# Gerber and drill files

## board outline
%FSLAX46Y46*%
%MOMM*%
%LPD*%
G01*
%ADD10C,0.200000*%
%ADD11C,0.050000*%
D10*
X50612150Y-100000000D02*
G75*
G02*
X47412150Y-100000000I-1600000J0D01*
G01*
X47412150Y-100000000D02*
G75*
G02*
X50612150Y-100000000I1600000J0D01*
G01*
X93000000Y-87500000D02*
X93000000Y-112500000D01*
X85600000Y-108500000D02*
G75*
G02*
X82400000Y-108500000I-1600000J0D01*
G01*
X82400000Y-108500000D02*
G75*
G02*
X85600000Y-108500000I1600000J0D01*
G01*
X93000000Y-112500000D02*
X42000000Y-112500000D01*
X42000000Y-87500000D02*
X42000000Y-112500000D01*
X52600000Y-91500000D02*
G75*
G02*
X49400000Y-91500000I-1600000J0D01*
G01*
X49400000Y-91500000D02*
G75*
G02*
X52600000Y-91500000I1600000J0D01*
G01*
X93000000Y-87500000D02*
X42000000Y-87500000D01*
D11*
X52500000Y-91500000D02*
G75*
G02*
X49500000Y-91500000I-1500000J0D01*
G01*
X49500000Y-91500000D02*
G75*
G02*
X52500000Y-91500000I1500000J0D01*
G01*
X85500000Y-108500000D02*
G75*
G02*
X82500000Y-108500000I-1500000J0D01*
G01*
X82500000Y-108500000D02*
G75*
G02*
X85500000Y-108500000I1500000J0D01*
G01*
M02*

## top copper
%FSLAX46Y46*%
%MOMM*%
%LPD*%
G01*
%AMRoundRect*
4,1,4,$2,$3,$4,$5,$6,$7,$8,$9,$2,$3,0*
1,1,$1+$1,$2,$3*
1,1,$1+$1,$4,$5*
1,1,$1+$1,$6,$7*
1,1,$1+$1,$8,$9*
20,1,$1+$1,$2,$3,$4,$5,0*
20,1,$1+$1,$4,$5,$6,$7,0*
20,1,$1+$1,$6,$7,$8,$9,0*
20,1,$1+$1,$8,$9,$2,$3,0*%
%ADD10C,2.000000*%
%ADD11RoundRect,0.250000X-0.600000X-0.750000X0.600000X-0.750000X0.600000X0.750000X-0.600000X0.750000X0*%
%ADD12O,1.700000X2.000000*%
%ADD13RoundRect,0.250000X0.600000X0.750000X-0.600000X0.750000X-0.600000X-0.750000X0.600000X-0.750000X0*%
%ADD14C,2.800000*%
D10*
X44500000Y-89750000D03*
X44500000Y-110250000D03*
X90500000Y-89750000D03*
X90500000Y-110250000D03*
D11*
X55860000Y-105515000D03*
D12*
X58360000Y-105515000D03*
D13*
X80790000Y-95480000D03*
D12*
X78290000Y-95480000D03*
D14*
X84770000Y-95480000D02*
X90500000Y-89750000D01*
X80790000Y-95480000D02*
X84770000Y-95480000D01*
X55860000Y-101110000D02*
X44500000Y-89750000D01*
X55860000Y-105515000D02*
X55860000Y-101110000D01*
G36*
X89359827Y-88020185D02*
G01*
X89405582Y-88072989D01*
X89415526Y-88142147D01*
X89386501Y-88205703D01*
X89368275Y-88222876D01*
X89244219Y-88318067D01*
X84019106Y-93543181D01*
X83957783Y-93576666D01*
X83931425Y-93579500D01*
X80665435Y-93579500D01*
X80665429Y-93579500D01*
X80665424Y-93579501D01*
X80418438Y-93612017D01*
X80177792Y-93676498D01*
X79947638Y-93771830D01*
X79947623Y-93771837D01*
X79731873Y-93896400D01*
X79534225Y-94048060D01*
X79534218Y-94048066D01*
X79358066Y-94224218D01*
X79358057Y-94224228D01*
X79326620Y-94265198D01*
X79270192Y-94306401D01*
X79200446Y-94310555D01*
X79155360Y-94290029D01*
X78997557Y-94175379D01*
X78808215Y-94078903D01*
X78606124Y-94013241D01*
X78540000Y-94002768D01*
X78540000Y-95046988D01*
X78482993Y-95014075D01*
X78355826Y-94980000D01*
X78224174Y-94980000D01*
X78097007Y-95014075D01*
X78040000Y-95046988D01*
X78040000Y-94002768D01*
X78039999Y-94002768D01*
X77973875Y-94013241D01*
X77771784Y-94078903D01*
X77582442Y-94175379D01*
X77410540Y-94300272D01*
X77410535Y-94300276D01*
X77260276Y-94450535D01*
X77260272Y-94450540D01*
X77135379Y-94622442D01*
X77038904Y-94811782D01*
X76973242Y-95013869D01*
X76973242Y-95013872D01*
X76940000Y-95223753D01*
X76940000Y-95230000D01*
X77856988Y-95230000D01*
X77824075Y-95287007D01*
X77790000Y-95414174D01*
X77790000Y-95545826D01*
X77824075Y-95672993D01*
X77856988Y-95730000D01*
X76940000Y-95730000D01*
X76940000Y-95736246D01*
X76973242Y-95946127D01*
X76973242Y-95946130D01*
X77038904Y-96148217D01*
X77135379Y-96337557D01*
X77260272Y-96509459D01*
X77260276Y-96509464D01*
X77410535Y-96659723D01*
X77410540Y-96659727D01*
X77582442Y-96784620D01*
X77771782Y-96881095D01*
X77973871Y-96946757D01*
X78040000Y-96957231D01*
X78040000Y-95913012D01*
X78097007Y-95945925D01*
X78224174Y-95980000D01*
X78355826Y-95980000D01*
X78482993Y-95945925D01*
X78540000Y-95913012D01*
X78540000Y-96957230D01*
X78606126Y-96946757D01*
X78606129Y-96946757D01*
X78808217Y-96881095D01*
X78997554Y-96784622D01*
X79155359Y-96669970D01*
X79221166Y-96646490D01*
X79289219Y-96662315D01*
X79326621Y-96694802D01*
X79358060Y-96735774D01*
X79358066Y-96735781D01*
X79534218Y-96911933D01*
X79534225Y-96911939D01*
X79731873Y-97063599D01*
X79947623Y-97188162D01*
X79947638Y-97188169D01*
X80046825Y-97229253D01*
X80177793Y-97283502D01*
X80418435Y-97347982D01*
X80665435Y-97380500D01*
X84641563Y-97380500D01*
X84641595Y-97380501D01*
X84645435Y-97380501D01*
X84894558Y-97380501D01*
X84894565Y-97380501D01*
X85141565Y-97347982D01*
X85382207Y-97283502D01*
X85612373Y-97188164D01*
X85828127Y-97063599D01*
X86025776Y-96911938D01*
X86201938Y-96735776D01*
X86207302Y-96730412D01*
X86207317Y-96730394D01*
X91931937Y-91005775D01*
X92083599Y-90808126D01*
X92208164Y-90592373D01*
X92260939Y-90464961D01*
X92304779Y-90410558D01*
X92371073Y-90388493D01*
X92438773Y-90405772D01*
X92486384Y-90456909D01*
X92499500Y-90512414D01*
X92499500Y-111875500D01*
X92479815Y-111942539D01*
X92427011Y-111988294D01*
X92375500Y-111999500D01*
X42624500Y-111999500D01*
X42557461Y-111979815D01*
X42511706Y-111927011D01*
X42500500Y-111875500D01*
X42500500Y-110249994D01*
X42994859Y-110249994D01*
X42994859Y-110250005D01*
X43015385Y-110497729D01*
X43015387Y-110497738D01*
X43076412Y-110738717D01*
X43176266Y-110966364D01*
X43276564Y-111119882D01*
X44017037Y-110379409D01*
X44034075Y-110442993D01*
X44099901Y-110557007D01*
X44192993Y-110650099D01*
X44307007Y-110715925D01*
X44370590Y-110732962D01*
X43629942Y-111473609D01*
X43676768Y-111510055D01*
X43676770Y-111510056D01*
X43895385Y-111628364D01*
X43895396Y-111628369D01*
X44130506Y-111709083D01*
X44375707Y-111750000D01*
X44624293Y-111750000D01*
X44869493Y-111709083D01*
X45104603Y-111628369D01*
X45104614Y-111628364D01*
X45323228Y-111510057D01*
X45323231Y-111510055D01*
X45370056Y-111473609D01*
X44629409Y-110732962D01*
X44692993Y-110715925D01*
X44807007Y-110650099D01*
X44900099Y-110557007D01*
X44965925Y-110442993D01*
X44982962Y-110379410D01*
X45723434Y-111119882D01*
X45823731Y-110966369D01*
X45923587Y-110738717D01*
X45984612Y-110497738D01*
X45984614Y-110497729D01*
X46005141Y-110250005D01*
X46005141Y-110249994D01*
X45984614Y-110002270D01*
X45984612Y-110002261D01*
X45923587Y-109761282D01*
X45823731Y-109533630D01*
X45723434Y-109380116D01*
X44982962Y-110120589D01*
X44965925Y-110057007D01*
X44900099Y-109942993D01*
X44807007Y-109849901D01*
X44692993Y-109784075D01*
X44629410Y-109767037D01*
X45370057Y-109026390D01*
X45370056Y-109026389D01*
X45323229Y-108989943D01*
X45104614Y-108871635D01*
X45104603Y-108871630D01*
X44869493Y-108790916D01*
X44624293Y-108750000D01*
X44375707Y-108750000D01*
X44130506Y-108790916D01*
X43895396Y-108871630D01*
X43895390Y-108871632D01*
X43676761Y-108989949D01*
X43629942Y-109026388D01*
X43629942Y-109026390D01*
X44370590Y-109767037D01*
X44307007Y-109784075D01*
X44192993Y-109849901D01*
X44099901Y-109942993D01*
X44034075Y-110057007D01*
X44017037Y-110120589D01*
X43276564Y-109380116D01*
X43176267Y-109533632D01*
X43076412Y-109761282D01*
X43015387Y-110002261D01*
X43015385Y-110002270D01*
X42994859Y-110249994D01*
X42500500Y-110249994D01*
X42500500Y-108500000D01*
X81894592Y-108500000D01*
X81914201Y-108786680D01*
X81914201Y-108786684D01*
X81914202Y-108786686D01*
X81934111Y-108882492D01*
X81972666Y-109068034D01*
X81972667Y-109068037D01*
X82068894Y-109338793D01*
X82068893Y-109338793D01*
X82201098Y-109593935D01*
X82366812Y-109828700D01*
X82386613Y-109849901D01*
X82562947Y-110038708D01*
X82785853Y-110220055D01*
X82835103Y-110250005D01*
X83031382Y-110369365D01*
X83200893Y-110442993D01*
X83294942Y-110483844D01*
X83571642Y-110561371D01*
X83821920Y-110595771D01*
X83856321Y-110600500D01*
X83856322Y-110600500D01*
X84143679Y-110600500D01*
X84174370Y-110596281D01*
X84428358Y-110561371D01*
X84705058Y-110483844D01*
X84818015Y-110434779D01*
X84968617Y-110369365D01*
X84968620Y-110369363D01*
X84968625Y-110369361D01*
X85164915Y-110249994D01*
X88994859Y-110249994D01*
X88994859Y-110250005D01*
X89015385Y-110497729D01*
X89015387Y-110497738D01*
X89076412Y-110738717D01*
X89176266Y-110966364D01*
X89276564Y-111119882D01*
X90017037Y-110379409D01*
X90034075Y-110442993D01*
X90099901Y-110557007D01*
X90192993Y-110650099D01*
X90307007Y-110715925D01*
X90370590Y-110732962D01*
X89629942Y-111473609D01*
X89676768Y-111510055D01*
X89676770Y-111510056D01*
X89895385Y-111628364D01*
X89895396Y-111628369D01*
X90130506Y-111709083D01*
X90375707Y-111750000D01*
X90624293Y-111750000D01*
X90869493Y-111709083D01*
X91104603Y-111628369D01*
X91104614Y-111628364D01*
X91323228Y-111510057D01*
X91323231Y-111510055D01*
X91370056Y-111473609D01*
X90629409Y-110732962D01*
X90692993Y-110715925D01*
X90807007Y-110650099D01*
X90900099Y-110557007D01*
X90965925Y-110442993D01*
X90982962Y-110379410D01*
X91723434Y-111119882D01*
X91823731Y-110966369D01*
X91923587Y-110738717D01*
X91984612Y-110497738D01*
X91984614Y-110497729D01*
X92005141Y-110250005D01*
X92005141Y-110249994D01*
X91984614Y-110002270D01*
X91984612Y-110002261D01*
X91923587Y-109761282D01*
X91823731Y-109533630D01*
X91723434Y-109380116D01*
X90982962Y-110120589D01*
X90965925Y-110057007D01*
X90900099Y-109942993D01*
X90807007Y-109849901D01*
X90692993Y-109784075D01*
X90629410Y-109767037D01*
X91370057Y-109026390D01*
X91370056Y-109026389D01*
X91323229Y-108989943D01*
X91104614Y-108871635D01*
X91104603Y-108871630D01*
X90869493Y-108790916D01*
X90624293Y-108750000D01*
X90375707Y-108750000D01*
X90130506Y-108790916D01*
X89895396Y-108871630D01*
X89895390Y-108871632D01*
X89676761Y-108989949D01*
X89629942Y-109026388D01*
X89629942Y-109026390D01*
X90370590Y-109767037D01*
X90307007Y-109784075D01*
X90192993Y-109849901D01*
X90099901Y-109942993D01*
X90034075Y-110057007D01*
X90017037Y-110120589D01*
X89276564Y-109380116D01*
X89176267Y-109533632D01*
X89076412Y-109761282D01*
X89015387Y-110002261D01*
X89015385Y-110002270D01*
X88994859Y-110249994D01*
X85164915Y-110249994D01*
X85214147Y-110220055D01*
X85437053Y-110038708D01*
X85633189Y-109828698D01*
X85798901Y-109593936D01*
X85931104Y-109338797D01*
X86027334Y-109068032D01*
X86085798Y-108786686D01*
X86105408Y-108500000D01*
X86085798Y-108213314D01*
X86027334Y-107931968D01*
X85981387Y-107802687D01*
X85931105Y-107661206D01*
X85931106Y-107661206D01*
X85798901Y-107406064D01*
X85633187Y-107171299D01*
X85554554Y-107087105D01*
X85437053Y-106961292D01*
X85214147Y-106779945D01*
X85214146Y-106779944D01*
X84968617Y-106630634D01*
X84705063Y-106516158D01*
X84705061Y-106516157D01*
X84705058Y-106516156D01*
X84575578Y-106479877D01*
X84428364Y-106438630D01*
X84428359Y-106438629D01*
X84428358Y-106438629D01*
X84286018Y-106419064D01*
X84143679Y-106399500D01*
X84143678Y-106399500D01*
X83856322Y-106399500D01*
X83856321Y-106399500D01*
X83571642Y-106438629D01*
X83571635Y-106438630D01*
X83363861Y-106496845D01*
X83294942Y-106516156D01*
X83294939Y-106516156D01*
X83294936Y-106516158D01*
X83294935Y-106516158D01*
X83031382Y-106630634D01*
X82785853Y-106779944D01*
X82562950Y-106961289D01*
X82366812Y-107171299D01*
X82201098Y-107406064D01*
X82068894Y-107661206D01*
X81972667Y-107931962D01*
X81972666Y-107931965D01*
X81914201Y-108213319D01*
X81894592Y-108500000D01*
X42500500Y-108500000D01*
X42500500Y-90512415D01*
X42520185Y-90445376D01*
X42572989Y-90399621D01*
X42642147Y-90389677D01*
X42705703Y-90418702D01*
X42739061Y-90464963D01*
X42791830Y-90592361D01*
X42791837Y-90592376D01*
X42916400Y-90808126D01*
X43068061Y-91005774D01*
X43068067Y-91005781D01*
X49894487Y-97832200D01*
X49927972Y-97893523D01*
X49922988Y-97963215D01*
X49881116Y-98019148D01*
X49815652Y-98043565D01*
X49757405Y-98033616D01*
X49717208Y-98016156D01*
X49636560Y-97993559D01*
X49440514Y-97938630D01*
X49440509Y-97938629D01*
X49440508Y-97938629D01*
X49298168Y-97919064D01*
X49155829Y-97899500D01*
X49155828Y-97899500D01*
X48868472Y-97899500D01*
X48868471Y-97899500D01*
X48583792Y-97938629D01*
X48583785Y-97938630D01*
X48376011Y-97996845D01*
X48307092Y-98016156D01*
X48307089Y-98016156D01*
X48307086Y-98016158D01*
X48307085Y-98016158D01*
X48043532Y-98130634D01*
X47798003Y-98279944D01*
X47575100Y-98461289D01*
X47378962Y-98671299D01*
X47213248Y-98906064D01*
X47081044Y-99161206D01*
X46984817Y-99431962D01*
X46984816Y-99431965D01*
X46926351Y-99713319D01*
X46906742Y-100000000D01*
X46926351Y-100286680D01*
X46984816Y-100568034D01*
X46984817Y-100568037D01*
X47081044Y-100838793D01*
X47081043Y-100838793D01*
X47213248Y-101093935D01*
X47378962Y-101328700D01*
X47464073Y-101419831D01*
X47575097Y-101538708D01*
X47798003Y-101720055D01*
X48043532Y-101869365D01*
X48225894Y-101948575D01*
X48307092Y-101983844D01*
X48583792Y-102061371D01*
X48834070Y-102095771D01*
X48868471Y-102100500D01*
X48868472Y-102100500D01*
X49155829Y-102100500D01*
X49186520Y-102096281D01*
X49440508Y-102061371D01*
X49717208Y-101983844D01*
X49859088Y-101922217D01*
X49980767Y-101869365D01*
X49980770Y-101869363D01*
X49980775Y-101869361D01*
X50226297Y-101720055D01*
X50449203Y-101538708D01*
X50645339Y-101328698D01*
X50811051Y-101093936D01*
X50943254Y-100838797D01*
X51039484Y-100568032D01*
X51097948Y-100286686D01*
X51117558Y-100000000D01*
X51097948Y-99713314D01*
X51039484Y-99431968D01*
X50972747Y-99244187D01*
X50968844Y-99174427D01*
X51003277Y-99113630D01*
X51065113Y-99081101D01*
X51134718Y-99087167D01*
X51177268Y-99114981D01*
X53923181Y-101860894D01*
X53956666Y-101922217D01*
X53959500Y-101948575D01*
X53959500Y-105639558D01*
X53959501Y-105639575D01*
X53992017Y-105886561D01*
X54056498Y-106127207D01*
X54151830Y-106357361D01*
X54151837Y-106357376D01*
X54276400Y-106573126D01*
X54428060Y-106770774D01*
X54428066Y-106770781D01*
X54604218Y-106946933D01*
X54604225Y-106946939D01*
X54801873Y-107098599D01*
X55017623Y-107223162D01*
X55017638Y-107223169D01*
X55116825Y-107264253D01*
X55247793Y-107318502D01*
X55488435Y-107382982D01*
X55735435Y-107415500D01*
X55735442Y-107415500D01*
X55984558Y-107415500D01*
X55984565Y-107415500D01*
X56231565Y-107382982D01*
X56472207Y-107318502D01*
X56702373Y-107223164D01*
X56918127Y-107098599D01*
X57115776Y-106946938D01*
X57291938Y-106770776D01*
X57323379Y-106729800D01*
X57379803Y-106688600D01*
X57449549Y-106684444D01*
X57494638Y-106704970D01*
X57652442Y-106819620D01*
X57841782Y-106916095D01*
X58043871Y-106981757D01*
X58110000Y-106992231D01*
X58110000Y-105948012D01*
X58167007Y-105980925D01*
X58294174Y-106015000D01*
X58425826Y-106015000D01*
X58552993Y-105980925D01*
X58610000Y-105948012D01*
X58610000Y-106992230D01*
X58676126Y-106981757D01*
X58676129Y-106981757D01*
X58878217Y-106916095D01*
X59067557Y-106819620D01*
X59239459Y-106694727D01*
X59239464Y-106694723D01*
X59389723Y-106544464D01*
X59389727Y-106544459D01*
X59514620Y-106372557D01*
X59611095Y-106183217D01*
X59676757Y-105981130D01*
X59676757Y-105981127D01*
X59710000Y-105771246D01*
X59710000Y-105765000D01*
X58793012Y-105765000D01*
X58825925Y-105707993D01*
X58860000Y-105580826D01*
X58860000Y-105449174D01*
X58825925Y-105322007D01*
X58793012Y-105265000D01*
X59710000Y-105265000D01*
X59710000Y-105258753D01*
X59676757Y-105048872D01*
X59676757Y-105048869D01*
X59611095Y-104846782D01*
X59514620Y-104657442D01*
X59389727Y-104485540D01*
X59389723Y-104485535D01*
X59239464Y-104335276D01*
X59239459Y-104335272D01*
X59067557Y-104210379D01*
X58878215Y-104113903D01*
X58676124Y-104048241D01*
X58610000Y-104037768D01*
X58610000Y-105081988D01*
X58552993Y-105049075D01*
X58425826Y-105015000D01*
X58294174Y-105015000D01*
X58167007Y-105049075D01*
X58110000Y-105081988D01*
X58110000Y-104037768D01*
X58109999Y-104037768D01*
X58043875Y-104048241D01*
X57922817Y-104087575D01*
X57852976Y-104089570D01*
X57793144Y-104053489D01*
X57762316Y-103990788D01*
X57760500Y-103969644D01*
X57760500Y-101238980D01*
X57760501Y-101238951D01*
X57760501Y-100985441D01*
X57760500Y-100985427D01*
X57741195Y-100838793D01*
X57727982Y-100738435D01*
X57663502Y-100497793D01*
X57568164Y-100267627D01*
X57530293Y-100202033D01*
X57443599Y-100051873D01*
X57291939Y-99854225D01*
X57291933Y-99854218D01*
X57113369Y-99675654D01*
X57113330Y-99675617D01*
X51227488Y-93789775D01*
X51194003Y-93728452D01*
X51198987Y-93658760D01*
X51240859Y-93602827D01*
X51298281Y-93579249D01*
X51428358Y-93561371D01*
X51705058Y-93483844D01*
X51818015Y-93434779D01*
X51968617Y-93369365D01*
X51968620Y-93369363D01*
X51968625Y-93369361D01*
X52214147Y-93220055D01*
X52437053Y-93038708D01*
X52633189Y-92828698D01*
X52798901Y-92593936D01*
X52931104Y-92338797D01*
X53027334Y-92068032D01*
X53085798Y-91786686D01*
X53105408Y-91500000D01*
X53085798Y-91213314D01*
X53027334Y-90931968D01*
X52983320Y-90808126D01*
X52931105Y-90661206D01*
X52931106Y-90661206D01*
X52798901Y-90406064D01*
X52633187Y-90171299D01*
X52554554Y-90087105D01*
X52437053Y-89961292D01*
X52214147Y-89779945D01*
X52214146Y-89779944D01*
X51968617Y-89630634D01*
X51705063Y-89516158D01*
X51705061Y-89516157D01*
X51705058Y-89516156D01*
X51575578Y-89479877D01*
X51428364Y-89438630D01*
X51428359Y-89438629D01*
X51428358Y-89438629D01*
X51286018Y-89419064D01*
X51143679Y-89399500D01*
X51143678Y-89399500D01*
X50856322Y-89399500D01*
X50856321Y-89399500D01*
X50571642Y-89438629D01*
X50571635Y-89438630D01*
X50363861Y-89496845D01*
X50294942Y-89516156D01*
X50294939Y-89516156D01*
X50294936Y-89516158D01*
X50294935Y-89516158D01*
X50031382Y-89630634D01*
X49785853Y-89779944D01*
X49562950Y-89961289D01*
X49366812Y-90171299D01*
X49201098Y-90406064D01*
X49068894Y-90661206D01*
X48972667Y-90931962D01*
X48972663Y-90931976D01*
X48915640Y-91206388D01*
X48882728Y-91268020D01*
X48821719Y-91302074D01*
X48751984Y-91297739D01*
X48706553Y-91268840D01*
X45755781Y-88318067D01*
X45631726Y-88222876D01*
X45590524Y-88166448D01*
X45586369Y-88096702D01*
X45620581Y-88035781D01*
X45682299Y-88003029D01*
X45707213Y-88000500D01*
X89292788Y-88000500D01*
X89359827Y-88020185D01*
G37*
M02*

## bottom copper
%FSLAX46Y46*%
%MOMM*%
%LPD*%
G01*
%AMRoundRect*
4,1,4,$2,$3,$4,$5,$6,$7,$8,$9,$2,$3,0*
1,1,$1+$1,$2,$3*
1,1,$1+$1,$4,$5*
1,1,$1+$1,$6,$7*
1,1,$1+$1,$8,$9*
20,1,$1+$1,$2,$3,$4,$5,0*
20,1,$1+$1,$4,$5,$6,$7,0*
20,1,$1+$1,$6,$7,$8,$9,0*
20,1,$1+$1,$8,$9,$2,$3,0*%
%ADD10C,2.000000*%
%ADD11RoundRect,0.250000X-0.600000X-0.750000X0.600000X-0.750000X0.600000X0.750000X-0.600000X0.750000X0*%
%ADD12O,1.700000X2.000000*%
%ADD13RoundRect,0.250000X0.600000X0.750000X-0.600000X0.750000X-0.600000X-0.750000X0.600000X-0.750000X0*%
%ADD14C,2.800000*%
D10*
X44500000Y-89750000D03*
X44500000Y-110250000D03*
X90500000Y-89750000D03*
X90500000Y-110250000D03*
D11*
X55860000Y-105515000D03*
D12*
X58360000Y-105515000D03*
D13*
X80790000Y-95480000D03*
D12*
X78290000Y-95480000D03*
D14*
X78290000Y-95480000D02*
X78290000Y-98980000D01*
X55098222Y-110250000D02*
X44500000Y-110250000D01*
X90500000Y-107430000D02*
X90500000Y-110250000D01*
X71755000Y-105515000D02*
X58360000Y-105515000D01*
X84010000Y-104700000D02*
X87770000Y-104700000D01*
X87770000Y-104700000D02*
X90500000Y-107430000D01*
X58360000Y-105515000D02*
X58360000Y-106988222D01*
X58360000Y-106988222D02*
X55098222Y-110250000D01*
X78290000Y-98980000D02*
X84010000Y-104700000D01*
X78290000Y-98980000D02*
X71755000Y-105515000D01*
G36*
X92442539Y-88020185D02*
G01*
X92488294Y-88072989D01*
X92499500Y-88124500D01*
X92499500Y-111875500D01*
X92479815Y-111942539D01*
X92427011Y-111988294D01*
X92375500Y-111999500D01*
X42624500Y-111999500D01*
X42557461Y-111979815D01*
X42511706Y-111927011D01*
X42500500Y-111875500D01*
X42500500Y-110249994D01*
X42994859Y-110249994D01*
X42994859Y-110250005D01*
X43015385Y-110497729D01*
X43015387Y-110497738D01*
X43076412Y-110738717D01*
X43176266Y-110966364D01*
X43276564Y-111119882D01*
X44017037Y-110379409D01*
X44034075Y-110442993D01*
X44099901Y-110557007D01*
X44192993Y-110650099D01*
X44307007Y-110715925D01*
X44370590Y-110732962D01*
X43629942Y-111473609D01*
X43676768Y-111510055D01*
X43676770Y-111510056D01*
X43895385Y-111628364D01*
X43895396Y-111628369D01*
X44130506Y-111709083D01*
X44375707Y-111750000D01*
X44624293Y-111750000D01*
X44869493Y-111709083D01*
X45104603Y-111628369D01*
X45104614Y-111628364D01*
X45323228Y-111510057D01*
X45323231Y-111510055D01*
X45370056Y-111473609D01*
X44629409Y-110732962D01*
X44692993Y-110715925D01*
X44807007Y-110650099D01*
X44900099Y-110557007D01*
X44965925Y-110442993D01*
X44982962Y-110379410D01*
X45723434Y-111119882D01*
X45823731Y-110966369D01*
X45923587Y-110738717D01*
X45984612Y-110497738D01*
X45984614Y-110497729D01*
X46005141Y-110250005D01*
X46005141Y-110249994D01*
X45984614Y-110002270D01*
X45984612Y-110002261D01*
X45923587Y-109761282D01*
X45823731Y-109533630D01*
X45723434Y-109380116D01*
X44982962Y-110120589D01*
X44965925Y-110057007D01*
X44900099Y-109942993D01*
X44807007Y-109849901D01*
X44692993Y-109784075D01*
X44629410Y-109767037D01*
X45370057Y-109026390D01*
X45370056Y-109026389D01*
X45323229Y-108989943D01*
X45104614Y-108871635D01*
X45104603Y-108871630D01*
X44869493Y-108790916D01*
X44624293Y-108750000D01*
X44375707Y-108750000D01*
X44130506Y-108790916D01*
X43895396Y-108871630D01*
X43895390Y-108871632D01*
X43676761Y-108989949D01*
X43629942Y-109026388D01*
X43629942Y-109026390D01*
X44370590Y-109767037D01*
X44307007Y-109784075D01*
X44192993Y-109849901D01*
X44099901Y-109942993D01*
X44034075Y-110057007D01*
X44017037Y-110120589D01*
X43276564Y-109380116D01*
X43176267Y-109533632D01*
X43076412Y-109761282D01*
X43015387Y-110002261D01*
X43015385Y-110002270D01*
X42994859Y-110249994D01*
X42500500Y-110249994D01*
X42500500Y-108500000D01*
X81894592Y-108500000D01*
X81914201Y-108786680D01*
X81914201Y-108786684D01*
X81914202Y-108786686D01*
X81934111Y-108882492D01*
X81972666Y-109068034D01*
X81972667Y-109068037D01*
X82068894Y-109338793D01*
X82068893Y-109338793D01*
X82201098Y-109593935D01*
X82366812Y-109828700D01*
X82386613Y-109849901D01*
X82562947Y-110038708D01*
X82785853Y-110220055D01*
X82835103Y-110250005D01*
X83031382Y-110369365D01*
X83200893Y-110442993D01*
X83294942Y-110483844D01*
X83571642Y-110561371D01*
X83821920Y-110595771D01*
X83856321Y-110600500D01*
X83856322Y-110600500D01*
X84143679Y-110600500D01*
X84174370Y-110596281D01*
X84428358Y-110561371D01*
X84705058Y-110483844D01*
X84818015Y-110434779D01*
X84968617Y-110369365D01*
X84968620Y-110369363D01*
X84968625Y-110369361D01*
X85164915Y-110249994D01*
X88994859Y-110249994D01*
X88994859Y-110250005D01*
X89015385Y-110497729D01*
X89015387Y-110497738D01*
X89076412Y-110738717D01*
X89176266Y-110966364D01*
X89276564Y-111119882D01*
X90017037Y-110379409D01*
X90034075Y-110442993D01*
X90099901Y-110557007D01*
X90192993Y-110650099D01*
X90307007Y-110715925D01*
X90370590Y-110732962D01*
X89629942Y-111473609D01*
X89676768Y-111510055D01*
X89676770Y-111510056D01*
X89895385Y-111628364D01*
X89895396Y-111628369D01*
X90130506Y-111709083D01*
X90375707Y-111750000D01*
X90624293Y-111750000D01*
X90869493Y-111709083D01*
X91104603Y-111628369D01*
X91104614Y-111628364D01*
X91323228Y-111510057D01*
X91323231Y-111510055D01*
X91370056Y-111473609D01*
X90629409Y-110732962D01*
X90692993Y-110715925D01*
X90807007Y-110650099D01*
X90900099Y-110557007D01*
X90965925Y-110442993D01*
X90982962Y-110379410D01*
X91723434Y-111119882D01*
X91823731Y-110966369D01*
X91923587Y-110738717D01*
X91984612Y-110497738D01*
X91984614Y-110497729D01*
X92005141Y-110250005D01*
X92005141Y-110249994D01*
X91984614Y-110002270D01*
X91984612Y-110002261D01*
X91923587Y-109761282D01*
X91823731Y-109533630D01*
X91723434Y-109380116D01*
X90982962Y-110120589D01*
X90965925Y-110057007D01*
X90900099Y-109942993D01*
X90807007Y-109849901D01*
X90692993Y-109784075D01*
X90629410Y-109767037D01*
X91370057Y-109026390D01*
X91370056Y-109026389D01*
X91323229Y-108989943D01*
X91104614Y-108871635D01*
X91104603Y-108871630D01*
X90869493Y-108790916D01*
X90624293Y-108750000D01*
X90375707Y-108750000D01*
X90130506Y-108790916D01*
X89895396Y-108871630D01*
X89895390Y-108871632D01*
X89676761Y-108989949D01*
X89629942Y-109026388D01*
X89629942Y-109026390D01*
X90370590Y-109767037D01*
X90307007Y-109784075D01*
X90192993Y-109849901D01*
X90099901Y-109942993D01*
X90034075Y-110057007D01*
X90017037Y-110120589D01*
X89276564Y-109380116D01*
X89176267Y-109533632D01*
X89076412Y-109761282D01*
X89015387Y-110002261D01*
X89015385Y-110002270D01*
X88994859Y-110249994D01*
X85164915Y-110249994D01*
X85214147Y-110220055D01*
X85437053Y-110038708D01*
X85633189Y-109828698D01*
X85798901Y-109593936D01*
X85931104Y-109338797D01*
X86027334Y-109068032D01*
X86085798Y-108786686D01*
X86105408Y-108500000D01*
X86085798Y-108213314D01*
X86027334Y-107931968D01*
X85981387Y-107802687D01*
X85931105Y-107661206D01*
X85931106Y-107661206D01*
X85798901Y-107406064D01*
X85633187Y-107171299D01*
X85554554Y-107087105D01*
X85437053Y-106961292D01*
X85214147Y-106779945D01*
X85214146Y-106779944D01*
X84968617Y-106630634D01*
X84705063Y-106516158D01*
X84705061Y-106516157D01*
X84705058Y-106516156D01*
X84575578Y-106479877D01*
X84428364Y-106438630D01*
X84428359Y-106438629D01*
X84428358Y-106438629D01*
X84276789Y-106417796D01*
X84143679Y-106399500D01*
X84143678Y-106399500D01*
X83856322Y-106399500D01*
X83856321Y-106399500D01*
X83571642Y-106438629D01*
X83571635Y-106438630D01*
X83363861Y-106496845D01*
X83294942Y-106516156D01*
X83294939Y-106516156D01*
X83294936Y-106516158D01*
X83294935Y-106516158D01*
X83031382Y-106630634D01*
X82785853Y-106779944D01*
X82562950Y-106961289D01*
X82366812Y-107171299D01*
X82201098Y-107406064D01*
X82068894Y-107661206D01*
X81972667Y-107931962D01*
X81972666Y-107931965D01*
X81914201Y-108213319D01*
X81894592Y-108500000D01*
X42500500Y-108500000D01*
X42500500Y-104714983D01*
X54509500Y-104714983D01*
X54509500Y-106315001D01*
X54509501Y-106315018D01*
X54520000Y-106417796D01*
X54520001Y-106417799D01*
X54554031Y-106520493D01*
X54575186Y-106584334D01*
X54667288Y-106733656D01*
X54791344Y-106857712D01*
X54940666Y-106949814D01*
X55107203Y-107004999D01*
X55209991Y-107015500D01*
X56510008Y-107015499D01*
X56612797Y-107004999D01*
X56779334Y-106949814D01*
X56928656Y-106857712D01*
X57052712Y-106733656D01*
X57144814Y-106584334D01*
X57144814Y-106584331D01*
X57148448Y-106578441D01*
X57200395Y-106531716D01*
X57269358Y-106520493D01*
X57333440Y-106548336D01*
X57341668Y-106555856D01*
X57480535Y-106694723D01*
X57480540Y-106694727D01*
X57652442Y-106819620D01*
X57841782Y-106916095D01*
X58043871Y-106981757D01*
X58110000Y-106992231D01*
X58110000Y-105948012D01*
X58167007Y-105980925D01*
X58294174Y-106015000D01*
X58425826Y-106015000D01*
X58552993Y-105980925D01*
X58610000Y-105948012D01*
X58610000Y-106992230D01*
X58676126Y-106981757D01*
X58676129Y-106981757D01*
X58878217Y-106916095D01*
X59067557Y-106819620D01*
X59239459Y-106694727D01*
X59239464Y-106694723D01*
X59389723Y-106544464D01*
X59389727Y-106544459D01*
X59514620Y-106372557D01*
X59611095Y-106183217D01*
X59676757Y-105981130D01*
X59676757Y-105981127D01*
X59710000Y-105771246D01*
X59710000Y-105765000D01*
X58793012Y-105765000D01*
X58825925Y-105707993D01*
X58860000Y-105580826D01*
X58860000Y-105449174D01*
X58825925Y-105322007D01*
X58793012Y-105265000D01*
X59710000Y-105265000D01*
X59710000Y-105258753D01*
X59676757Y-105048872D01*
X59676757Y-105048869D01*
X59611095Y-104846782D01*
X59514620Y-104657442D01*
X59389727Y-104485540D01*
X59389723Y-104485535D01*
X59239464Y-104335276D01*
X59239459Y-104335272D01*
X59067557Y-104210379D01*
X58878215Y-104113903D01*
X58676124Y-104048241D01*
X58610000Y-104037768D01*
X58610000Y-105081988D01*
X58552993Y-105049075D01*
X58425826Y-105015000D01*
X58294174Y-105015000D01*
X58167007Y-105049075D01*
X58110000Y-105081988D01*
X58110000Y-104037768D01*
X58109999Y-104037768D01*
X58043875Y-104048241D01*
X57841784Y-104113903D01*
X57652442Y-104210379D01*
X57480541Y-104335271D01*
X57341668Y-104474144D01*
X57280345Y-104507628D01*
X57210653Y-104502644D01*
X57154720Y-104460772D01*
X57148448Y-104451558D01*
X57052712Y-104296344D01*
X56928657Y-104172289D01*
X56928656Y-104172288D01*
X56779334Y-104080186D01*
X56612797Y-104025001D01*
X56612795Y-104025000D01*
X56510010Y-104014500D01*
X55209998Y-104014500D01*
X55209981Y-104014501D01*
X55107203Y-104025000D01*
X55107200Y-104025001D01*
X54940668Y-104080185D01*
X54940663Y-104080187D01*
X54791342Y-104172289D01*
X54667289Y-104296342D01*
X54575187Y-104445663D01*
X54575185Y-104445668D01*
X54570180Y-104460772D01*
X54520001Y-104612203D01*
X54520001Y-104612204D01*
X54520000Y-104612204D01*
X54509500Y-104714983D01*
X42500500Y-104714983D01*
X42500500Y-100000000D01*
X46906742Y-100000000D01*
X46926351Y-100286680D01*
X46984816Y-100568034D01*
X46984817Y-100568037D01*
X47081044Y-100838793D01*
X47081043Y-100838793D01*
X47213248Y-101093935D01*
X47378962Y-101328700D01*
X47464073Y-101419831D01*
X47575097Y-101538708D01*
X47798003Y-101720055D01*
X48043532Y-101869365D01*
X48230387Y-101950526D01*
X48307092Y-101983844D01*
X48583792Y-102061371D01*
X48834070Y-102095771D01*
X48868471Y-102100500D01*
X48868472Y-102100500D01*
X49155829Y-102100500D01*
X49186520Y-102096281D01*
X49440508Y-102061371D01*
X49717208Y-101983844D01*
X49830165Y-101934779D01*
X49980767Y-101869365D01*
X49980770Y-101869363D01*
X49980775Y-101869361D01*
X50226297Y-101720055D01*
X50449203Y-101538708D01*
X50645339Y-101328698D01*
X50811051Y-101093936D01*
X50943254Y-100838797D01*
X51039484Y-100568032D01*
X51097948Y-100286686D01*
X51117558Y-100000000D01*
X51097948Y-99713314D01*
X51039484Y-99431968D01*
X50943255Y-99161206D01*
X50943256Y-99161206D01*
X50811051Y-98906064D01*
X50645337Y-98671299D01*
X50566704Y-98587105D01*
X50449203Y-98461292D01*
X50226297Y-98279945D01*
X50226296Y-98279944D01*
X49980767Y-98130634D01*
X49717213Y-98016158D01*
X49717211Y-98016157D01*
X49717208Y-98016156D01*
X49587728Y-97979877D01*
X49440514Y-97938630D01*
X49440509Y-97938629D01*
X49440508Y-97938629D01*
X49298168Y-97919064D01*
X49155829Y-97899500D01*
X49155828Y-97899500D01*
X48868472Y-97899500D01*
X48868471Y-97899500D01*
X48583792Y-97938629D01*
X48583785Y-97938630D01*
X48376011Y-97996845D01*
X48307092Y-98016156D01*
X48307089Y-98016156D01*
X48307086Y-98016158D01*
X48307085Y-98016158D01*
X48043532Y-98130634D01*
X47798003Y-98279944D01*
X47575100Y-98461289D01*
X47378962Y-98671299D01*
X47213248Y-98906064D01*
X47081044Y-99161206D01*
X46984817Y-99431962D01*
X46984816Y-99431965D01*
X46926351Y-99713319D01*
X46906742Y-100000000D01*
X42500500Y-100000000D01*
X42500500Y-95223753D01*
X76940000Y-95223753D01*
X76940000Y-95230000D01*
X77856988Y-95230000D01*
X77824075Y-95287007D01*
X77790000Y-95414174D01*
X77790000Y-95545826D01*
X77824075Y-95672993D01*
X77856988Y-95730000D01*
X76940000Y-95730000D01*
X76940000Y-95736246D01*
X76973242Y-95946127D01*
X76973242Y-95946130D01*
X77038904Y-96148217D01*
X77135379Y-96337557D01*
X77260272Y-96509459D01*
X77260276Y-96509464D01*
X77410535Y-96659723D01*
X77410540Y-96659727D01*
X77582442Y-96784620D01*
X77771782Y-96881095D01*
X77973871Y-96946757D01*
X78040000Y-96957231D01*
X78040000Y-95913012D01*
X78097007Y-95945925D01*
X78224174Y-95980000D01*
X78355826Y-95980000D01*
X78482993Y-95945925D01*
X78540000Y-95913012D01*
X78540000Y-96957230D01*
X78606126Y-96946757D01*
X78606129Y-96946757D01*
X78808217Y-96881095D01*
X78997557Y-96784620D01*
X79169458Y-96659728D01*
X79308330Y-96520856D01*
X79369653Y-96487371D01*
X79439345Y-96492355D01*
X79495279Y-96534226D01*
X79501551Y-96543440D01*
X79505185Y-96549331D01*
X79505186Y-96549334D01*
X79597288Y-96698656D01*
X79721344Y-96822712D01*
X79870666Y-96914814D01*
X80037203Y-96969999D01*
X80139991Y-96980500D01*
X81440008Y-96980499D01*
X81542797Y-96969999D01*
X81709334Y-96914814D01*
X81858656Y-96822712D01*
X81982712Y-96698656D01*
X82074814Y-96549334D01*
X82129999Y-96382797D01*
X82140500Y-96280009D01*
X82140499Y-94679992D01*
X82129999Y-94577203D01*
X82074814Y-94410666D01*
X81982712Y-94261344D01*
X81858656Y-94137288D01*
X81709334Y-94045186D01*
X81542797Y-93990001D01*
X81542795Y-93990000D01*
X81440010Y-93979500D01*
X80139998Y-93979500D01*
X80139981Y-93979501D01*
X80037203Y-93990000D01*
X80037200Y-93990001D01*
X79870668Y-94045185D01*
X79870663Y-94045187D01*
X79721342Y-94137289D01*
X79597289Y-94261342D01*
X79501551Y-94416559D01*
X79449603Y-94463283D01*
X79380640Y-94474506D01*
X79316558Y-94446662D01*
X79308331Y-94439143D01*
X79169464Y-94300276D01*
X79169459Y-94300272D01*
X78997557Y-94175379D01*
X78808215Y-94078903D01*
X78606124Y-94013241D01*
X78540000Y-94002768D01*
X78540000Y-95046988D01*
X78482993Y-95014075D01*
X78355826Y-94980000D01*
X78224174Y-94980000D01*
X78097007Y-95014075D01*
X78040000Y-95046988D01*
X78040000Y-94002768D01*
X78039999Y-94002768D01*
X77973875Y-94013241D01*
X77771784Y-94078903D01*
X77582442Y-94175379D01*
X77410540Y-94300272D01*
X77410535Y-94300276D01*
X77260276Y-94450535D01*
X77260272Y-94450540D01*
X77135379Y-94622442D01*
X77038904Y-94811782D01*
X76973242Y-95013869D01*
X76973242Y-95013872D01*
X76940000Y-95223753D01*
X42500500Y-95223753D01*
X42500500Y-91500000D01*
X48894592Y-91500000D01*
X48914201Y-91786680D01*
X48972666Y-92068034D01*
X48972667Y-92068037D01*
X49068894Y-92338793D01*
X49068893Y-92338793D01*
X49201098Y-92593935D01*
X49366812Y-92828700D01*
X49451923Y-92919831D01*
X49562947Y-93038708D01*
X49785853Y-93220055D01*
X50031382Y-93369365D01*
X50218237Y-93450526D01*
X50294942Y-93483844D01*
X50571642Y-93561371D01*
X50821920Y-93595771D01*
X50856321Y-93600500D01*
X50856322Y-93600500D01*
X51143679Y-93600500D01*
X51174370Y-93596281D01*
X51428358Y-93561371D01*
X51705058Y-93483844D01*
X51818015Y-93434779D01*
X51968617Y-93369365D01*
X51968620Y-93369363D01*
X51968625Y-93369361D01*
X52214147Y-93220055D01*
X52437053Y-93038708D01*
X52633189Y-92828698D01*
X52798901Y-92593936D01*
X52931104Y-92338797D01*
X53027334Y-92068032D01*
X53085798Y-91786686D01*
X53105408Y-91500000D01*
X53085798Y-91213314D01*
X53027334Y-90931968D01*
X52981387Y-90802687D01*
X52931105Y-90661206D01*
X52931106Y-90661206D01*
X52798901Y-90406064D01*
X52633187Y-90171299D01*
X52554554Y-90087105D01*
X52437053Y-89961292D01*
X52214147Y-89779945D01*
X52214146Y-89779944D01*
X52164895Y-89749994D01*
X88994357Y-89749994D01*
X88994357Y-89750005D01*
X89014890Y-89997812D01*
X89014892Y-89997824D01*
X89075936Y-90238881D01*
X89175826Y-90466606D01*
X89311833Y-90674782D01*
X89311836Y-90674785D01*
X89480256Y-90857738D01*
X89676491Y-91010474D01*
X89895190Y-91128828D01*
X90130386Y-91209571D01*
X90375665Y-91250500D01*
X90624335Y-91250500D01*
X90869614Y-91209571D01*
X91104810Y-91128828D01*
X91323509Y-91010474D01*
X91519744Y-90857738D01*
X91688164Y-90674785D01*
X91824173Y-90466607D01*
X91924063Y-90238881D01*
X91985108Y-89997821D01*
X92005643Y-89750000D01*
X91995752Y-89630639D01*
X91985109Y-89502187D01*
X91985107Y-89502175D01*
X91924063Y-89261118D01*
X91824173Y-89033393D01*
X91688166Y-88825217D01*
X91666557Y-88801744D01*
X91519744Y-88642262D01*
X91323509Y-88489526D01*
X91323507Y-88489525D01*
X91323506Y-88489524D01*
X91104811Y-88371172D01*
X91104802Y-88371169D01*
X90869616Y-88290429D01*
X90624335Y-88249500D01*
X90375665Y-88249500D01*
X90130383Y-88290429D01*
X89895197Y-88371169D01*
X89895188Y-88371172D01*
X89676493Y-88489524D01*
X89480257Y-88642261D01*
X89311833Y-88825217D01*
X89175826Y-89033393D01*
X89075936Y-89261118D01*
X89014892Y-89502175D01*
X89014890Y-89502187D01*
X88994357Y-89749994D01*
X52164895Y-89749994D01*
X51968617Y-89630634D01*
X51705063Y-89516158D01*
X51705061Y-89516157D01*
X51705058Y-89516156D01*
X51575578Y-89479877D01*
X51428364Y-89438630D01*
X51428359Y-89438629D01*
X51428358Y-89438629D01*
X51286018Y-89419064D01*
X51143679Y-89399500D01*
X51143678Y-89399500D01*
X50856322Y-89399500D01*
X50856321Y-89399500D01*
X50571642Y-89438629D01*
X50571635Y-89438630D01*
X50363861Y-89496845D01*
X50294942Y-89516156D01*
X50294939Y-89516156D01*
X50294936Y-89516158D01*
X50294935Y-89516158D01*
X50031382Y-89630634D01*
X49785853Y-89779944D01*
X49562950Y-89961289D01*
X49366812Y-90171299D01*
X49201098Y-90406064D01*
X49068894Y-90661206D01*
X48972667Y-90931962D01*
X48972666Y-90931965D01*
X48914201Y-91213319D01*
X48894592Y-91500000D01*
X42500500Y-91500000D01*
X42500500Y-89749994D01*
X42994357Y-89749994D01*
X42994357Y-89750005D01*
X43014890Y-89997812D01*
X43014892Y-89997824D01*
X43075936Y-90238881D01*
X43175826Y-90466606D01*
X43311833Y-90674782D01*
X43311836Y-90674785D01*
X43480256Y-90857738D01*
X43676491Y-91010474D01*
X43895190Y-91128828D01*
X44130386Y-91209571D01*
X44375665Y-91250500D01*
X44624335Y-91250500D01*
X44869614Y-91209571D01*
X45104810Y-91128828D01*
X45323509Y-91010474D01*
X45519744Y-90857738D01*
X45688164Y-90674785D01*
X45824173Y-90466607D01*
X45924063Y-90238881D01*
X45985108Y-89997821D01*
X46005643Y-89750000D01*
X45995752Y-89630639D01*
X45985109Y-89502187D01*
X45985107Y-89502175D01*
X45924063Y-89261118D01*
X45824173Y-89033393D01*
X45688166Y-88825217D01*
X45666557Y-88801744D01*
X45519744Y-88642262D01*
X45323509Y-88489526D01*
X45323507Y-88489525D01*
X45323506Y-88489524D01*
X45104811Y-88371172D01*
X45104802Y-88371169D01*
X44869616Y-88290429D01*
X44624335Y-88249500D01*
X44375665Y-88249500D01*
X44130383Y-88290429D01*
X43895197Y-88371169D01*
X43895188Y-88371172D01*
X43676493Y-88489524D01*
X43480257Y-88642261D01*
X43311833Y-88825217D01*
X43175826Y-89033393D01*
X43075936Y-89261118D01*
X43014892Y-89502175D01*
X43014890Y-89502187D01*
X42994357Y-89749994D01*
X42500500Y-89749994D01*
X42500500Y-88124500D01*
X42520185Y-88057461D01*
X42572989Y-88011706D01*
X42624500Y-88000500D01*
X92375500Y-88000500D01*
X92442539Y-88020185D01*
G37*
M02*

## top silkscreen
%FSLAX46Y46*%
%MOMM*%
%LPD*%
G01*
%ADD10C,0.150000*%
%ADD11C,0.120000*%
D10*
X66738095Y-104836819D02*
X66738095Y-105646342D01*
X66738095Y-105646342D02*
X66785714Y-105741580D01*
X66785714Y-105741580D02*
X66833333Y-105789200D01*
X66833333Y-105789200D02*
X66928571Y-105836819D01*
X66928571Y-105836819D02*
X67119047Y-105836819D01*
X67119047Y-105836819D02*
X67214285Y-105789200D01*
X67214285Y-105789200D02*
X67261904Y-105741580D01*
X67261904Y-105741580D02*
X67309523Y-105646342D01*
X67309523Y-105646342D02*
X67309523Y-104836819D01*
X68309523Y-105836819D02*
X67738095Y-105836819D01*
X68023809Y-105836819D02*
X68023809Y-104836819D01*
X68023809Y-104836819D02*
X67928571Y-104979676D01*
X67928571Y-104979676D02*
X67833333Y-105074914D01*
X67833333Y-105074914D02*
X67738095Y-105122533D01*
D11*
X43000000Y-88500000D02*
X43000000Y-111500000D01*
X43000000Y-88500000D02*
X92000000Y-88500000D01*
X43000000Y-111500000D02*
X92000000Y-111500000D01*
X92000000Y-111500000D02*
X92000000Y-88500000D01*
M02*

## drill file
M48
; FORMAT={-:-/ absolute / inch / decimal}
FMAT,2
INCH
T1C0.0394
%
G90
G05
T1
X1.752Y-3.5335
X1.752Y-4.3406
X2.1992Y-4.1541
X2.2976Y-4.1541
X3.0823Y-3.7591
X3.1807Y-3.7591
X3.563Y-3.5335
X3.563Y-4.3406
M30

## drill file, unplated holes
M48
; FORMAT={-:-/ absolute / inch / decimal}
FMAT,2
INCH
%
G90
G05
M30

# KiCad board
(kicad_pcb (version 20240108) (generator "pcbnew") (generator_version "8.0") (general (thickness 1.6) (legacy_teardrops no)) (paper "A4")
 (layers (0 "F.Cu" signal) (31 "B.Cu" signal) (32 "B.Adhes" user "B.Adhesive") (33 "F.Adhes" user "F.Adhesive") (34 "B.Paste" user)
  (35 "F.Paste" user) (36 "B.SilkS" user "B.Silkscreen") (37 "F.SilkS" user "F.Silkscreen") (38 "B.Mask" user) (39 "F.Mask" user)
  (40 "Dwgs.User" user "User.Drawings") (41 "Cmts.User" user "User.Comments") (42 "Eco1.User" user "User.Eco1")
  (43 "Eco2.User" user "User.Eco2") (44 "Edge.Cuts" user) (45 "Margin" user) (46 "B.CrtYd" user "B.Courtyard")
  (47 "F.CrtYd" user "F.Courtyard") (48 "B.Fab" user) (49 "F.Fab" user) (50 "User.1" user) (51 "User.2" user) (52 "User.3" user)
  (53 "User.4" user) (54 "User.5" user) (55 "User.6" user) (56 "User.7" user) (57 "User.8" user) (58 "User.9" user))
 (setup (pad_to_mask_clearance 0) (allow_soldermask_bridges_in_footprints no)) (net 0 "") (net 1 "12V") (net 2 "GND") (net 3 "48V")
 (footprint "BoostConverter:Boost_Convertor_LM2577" (layer "F.Cu") (at 67.5 100)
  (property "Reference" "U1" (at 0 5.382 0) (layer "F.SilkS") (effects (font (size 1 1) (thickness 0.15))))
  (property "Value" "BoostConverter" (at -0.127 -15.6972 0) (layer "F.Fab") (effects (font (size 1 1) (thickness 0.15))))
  (fp_line (start -24.5 -11.5) (end -24.5 11.5) (stroke (width 0.12) (type solid)) (layer "F.SilkS"))
  (fp_line (start -24.5 -11.5) (end 24.5 -11.5) (stroke (width 0.12) (type solid)) (layer "F.SilkS"))
  (fp_line (start -24.5 11.5) (end 24.5 11.5) (stroke (width 0.12) (type solid)) (layer "F.SilkS"))
  (fp_line (start 24.5 11.5) (end 24.5 -11.5) (stroke (width 0.12) (type solid)) (layer "F.SilkS"))
  (fp_circle (center -16.5 -8.5) (end -15 -8.5) (stroke (width 0.05) (type default)) (fill none) (layer "Edge.Cuts"))
  (fp_circle (center 16.5 8.5) (end 18 8.5) (stroke (width 0.05) (type default)) (fill none) (layer "Edge.Cuts"))
  (pad "1" thru_hole circle (at -23 -10.25) (size 2 2) (drill 1) (layers "*.Cu" "*.Mask") (remove_unused_layers no) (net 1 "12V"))
  (pad "2" thru_hole circle (at -23 10.25) (size 2 2) (drill 1) (layers "*.Cu" "*.Mask") (remove_unused_layers no) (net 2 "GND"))
  (pad "3" thru_hole circle (at 23 -10.25) (size 2 2) (drill 1) (layers "*.Cu" "*.Mask") (remove_unused_layers no) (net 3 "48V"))
  (pad "4" thru_hole circle (at 23 10.25) (size 2 2) (drill 1) (layers "*.Cu" "*.Mask") (remove_unused_layers no) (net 2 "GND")))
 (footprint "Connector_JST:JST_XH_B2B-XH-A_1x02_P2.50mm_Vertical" (layer "B.Cu") (at 55.86 105.515)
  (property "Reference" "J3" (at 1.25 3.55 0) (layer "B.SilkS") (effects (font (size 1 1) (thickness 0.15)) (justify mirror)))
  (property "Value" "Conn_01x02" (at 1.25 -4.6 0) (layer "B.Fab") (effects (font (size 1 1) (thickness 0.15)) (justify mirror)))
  (pad "1" thru_hole roundrect (at 0 0) (size 1.7 2) (drill 1) (layers "*.Cu" "*.Mask") (remove_unused_layers no)
   (roundrect_rratio 0.147059) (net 1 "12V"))
  (pad "2" thru_hole oval (at 2.5 0) (size 1.7 2) (drill 1) (layers "*.Cu" "*.Mask") (remove_unused_layers no) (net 2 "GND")))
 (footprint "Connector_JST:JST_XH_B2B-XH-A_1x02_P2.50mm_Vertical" (layer "B.Cu") (at 80.79 95.48 180)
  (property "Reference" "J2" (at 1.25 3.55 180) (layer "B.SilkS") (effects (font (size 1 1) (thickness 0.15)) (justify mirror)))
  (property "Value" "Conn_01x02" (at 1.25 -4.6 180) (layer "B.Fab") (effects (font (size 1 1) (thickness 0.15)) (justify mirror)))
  (pad "1" thru_hole roundrect (at 0 0 180) (size 1.7 2) (drill 1) (layers "*.Cu" "*.Mask") (remove_unused_layers no)
   (roundrect_rratio 0.147059) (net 3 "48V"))
  (pad "2" thru_hole oval (at 2.5 0 180) (size 1.7 2) (drill 1) (layers "*.Cu" "*.Mask") (remove_unused_layers no) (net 2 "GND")))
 (gr_circle (center 49.01215 100) (end 50.61215 100) (stroke (width 0.2) (type default)) (fill none) (layer "Edge.Cuts"))
 (gr_line (start 93 87.5) (end 93 112.5) (stroke (width 0.2) (type default)) (layer "Edge.Cuts"))
 (gr_circle (center 84 108.5) (end 85.6 108.5) (stroke (width 0.2) (type default)) (fill none) (layer "Edge.Cuts"))
 (gr_line (start 93 112.5) (end 42 112.5) (stroke (width 0.2) (type default)) (layer "Edge.Cuts"))
 (gr_line (start 42 87.5) (end 42 112.5) (stroke (width 0.2) (type default)) (layer "Edge.Cuts"))
 (gr_circle (center 51 91.5) (end 52.6 91.5) (stroke (width 0.2) (type default)) (fill none) (layer "Edge.Cuts"))
 (gr_line (start 93 87.5) (end 42 87.5) (stroke (width 0.2) (type default)) (layer "Edge.Cuts"))
 (segment (start 84.77 95.48) (end 90.5 89.75) (width 2.8) (layer "F.Cu") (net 3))
 (segment (start 80.79 95.48) (end 84.77 95.48) (width 2.8) (layer "F.Cu") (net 3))
 (segment (start 78.29 95.48) (end 78.29 98.98) (width 2.8) (layer "B.Cu") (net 2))
 (segment (start 55.098222 110.25) (end 44.5 110.25) (width 2.8) (layer "B.Cu") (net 2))
 (segment (start 90.5 107.43) (end 90.5 110.25) (width 2.8) (layer "B.Cu") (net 2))
 (segment (start 71.755 105.515) (end 58.36 105.515) (width 2.8) (layer "B.Cu") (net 2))
 (segment (start 84.01 104.7) (end 87.77 104.7) (width 2.8) (layer "B.Cu") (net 2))
 (segment (start 87.77 104.7) (end 90.5 107.43) (width 2.8) (layer "B.Cu") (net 2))
 (segment (start 58.36 105.515) (end 58.36 106.988222) (width 2.8) (layer "B.Cu") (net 2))
 (segment (start 58.36 106.988222) (end 55.098222 110.25) (width 2.8) (layer "B.Cu") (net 2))
 (segment (start 78.29 98.98) (end 84.01 104.7) (width 2.8) (layer "B.Cu") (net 2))
 (segment (start 78.29 98.98) (end 71.755 105.515) (width 2.8) (layer "B.Cu") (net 2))
 (segment (start 55.86 101.11) (end 44.5 89.75) (width 2.8) (layer "F.Cu") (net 1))
 (segment (start 55.86 105.515) (end 55.86 101.11) (width 2.8) (layer "F.Cu") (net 1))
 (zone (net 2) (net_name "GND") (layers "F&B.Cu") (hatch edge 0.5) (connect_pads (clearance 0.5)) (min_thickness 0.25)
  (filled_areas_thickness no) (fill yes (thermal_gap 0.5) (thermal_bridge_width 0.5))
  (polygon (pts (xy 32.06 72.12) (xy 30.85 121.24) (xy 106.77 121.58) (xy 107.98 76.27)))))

